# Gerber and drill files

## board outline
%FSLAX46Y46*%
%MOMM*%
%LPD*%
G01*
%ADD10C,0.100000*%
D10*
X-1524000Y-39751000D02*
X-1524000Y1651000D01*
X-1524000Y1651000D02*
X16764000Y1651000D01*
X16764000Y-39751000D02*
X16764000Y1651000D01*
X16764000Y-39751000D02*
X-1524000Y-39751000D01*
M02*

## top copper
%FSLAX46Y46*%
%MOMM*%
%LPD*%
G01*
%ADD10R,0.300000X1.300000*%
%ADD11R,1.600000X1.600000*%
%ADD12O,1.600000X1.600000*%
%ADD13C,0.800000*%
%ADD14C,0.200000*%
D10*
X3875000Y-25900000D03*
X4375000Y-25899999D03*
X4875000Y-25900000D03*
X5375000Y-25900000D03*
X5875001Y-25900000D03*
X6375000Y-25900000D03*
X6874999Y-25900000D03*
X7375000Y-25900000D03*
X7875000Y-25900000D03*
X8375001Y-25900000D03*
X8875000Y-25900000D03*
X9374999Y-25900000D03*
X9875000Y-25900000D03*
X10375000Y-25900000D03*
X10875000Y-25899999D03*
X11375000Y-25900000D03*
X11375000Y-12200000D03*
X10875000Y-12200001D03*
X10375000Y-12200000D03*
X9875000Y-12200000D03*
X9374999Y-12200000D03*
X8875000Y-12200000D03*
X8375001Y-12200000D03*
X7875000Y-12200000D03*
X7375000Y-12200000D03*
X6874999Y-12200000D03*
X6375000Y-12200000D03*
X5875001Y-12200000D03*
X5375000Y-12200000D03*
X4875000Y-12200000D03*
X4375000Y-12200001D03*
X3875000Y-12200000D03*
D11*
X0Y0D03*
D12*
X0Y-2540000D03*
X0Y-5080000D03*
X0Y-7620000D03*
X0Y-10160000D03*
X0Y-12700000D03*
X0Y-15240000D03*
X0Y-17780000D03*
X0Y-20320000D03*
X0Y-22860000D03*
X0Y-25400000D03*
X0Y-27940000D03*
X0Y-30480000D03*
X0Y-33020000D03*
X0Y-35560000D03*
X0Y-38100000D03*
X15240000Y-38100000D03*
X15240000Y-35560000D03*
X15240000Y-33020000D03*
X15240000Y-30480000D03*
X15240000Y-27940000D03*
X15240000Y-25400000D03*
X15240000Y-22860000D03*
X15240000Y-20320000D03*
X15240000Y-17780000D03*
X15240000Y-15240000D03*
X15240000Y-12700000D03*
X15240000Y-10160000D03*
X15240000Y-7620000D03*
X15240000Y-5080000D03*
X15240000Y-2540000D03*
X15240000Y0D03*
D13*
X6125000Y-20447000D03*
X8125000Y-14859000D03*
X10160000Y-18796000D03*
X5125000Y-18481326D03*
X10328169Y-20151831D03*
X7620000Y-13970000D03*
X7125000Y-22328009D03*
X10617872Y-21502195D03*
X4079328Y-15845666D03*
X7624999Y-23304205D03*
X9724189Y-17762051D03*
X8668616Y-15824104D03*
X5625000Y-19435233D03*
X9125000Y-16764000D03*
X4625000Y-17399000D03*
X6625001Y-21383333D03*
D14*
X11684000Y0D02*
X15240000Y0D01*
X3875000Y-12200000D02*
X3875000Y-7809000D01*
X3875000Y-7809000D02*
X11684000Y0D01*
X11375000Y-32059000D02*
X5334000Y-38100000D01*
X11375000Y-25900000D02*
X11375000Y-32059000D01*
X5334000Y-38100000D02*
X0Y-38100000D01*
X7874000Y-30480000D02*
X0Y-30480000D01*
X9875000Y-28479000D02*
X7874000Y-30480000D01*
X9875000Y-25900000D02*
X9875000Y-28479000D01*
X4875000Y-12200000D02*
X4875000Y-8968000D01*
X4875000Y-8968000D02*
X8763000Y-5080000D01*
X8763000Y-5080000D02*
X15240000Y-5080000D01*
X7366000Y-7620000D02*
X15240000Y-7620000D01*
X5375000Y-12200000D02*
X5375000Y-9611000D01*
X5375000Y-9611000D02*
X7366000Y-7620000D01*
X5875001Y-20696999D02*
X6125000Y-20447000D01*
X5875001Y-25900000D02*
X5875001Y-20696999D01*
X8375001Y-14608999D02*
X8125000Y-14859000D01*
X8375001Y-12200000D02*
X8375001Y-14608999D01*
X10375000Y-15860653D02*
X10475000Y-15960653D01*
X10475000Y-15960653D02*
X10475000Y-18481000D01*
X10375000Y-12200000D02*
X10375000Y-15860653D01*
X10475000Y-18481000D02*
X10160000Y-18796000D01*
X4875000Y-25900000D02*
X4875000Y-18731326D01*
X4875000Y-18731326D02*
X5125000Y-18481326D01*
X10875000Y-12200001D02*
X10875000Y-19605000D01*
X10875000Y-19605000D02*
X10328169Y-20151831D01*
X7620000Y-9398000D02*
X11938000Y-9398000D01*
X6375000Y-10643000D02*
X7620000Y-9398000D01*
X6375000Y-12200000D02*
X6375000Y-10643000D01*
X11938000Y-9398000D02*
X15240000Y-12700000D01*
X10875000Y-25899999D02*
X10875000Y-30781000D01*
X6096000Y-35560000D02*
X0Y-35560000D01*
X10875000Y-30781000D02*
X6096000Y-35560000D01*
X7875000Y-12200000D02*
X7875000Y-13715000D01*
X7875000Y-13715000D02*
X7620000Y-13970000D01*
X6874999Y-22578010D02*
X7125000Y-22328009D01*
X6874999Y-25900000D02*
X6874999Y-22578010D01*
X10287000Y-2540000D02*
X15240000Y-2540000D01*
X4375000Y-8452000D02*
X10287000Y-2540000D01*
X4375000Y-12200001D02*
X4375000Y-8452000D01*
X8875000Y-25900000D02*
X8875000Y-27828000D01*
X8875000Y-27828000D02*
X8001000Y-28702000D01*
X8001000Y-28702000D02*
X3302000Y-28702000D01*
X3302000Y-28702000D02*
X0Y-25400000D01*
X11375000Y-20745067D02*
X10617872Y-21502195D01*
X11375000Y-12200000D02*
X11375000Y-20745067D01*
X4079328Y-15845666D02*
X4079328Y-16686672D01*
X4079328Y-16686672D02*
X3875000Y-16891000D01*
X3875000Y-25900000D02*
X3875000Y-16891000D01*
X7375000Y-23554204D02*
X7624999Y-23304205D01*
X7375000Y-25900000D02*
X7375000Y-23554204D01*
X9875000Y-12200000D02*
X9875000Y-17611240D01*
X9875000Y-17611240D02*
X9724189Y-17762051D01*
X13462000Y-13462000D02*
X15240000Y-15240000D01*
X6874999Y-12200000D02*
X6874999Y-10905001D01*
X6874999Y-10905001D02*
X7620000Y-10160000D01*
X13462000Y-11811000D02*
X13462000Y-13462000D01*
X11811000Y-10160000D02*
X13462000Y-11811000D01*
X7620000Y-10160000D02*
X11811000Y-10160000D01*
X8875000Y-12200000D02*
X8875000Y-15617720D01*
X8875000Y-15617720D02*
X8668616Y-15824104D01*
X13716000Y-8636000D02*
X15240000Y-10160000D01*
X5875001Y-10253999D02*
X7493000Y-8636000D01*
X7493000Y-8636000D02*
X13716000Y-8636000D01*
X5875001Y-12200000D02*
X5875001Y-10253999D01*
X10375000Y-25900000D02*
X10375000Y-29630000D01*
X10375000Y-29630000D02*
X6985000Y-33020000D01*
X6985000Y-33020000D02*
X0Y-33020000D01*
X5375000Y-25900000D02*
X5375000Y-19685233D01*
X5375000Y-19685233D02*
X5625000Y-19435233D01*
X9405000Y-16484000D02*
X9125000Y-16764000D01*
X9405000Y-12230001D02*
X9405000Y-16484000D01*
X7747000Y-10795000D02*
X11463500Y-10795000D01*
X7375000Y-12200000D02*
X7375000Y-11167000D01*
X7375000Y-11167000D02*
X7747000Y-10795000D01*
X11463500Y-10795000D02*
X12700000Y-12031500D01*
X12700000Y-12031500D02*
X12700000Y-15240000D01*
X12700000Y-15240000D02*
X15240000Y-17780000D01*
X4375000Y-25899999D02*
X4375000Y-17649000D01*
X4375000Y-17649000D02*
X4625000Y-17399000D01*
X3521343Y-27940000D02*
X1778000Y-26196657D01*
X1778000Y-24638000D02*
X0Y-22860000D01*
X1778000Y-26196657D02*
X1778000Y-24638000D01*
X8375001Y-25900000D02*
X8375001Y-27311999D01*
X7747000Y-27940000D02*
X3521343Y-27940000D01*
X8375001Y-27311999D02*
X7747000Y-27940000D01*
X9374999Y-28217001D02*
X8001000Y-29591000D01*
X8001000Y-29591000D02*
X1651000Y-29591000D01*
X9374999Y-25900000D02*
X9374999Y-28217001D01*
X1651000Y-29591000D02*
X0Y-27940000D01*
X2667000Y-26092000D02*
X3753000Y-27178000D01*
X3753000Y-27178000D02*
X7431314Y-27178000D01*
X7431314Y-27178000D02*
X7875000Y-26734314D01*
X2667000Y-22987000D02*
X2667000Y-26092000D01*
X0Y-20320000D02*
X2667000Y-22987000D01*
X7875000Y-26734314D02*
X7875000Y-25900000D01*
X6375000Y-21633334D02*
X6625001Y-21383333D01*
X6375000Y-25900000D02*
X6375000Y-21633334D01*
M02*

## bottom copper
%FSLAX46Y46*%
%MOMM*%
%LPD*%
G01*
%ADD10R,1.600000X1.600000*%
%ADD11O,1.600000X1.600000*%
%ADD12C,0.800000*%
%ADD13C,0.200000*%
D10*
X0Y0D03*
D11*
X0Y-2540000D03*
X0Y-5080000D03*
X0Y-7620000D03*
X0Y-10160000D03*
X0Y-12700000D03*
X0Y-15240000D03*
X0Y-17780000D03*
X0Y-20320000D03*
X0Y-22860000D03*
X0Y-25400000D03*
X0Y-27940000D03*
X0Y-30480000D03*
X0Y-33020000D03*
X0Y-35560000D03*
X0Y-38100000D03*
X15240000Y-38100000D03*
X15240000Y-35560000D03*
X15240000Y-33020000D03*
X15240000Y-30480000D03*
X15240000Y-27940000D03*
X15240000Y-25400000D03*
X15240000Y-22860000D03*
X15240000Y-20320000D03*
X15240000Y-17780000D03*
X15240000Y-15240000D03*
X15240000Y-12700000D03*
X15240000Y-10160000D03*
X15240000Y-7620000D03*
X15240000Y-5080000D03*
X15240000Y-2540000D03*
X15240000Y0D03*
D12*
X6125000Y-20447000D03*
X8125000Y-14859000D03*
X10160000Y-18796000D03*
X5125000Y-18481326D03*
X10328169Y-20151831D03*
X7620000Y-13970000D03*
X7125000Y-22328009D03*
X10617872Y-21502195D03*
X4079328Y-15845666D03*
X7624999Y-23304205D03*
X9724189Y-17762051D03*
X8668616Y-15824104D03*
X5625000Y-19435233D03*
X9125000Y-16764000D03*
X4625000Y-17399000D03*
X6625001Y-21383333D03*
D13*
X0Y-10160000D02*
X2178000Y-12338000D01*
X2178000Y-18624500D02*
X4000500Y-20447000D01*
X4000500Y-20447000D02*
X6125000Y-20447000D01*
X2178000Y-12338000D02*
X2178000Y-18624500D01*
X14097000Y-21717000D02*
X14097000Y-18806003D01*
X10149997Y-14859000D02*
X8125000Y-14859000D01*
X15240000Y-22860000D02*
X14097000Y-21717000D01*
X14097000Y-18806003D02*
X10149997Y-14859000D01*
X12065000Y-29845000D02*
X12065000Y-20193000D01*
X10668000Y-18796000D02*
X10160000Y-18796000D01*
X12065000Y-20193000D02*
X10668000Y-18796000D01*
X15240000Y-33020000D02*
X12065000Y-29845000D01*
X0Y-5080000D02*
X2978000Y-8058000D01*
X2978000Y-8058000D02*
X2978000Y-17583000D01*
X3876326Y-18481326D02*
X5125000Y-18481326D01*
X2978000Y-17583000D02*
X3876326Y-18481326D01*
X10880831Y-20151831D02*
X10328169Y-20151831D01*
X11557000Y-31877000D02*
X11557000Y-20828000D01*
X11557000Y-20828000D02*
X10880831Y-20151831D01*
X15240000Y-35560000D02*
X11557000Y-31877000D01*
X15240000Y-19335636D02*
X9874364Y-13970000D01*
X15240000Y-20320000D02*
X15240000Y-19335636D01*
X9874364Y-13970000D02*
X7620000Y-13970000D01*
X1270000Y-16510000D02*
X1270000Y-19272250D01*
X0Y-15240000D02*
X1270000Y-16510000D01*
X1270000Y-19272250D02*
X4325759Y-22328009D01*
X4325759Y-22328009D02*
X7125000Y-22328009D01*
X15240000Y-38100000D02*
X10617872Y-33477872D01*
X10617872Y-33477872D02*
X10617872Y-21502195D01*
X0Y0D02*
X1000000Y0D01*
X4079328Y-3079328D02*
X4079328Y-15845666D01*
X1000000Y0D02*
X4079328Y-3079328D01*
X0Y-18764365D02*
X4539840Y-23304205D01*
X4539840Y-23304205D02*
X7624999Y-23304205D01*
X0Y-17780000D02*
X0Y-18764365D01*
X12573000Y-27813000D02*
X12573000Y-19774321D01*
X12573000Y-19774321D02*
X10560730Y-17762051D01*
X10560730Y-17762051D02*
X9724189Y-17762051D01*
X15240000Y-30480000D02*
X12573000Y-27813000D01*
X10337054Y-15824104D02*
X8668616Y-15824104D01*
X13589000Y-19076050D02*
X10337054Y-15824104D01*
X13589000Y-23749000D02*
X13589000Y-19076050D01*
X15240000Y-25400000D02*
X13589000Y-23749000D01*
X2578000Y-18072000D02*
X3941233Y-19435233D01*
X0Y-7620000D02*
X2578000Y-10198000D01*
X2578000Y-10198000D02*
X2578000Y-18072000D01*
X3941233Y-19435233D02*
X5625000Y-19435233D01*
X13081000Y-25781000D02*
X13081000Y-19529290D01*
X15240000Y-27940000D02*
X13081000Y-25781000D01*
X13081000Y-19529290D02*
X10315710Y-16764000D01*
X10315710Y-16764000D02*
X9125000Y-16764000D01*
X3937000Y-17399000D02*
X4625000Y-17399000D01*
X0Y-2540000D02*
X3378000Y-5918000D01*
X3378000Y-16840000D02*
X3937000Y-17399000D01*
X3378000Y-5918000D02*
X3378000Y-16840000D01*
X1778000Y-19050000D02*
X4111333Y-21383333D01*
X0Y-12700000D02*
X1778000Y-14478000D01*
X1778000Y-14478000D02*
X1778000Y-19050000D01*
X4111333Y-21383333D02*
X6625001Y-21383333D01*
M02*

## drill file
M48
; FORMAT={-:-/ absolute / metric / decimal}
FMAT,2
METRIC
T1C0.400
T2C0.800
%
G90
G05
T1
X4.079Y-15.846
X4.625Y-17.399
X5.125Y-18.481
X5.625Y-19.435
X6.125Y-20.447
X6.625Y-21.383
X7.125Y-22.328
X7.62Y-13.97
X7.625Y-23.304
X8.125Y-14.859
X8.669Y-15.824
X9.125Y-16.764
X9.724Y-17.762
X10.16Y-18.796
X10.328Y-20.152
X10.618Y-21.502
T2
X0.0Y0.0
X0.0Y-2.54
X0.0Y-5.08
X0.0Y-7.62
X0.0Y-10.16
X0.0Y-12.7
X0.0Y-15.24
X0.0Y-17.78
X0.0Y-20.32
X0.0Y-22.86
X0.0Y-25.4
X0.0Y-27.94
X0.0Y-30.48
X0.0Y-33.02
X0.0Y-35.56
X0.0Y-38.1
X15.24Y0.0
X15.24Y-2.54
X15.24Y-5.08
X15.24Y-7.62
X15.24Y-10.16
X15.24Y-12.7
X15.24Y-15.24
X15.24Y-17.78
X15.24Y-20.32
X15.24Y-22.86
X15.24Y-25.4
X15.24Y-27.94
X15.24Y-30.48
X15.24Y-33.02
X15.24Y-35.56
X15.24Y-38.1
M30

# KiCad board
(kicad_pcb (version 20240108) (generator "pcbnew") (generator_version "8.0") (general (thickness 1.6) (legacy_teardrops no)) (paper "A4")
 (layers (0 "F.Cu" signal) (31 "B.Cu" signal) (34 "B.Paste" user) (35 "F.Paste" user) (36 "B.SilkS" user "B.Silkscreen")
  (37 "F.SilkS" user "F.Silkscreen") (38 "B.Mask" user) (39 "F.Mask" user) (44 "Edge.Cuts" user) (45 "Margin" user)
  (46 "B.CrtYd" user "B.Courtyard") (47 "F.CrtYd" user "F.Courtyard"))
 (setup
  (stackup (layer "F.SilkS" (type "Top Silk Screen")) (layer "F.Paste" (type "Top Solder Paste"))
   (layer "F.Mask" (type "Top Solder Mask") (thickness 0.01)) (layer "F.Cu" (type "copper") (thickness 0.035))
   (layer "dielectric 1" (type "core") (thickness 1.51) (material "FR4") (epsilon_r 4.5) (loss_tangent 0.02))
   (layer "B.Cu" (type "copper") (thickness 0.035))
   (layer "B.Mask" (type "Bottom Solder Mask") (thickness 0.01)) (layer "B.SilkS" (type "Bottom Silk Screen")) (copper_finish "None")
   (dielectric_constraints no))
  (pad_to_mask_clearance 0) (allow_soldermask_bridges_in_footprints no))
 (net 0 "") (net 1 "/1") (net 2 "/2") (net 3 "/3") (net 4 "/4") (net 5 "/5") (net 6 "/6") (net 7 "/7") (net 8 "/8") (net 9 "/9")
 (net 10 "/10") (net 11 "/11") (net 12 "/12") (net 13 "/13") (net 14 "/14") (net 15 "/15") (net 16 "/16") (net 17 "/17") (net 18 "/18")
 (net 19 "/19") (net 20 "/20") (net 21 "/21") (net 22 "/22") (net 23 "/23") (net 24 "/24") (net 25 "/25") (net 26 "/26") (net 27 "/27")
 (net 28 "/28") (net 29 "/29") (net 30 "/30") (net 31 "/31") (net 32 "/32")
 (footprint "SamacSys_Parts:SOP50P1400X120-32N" (layer "F.Cu") (at 7.625 19.05 90)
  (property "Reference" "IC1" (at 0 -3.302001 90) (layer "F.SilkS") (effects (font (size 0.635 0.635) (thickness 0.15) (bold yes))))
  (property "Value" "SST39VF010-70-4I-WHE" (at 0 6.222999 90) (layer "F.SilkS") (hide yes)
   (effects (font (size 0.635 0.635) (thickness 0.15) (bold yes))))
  (pad "1" smd rect (at -6.85 -3.75 180) (size 0.3 1.3) (layers "F.Cu" "F.Paste" "F.Mask") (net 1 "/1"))
  (pad "2" smd rect (at -6.849999 -3.25 180) (size 0.3 1.3) (layers "F.Cu" "F.Paste" "F.Mask") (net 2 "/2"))
  (pad "3" smd rect (at -6.85 -2.75 180) (size 0.3 1.3) (layers "F.Cu" "F.Paste" "F.Mask") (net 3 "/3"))
  (pad "4" smd rect (at -6.85 -2.25 180) (size 0.3 1.3) (layers "F.Cu" "F.Paste" "F.Mask") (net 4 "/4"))
  (pad "5" smd rect (at -6.85 -1.749999 180) (size 0.3 1.3) (layers "F.Cu" "F.Paste" "F.Mask") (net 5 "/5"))
  (pad "6" smd rect (at -6.85 -1.25 180) (size 0.3 1.3) (layers "F.Cu" "F.Paste" "F.Mask") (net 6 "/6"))
  (pad "7" smd rect (at -6.85 -0.750001 180) (size 0.3 1.3) (layers "F.Cu" "F.Paste" "F.Mask") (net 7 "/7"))
  (pad "8" smd rect (at -6.85 -0.25 180) (size 0.3 1.3) (layers "F.Cu" "F.Paste" "F.Mask") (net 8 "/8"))
  (pad "9" smd rect (at -6.85 0.25 180) (size 0.3 1.3) (layers "F.Cu" "F.Paste" "F.Mask") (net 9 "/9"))
  (pad "10" smd rect (at -6.85 0.750001 180) (size 0.3 1.3) (layers "F.Cu" "F.Paste" "F.Mask") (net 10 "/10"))
  (pad "11" smd rect (at -6.85 1.25 180) (size 0.3 1.3) (layers "F.Cu" "F.Paste" "F.Mask") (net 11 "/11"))
  (pad "12" smd rect (at -6.85 1.749999 180) (size 0.3 1.3) (layers "F.Cu" "F.Paste" "F.Mask") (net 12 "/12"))
  (pad "13" smd rect (at -6.85 2.25 180) (size 0.3 1.3) (layers "F.Cu" "F.Paste" "F.Mask") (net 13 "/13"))
  (pad "14" smd rect (at -6.85 2.75 180) (size 0.3 1.3) (layers "F.Cu" "F.Paste" "F.Mask") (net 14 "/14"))
  (pad "15" smd rect (at -6.849999 3.25 180) (size 0.3 1.3) (layers "F.Cu" "F.Paste" "F.Mask") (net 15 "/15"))
  (pad "16" smd rect (at -6.85 3.75 180) (size 0.3 1.3) (layers "F.Cu" "F.Paste" "F.Mask") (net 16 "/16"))
  (pad "17" smd rect (at 6.85 3.75 180) (size 0.3 1.3) (layers "F.Cu" "F.Paste" "F.Mask") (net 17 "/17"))
  (pad "18" smd rect (at 6.849999 3.25 180) (size 0.3 1.3) (layers "F.Cu" "F.Paste" "F.Mask") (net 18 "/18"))
  (pad "19" smd rect (at 6.85 2.75 180) (size 0.3 1.3) (layers "F.Cu" "F.Paste" "F.Mask") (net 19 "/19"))
  (pad "20" smd rect (at 6.85 2.25 180) (size 0.3 1.3) (layers "F.Cu" "F.Paste" "F.Mask") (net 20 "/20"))
  (pad "21" smd rect (at 6.85 1.749999 180) (size 0.3 1.3) (layers "F.Cu" "F.Paste" "F.Mask") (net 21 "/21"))
  (pad "22" smd rect (at 6.85 1.25 180) (size 0.3 1.3) (layers "F.Cu" "F.Paste" "F.Mask") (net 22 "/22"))
  (pad "23" smd rect (at 6.85 0.750001 180) (size 0.3 1.3) (layers "F.Cu" "F.Paste" "F.Mask") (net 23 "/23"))
  (pad "24" smd rect (at 6.85 0.25 180) (size 0.3 1.3) (layers "F.Cu" "F.Paste" "F.Mask") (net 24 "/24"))
  (pad "25" smd rect (at 6.85 -0.25 180) (size 0.3 1.3) (layers "F.Cu" "F.Paste" "F.Mask") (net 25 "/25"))
  (pad "26" smd rect (at 6.85 -0.750001 180) (size 0.3 1.3) (layers "F.Cu" "F.Paste" "F.Mask") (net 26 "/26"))
  (pad "27" smd rect (at 6.85 -1.25 180) (size 0.3 1.3) (layers "F.Cu" "F.Paste" "F.Mask") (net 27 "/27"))
  (pad "28" smd rect (at 6.85 -1.749999 180) (size 0.3 1.3) (layers "F.Cu" "F.Paste" "F.Mask") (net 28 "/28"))
  (pad "29" smd rect (at 6.85 -2.25 180) (size 0.3 1.3) (layers "F.Cu" "F.Paste" "F.Mask") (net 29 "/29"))
  (pad "30" smd rect (at 6.85 -2.75 180) (size 0.3 1.3) (layers "F.Cu" "F.Paste" "F.Mask") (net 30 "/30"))
  (pad "31" smd rect (at 6.849999 -3.25 180) (size 0.3 1.3) (layers "F.Cu" "F.Paste" "F.Mask") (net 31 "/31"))
  (pad "32" smd rect (at 6.85 -3.75 180) (size 0.3 1.3) (layers "F.Cu" "F.Paste" "F.Mask") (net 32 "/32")))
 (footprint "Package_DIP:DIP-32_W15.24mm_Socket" (layer "F.Cu") (at 0 0)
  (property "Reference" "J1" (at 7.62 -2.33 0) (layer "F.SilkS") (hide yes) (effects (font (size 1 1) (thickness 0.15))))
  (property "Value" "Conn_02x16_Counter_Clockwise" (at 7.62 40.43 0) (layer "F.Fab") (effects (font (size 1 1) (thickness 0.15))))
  (pad "1" thru_hole rect (at 0 0) (size 1.6 1.6) (drill 0.8) (layers "*.Cu" "*.Mask") (remove_unused_layers no) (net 1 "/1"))
  (pad "2" thru_hole oval (at 0 2.54) (size 1.6 1.6) (drill 0.8) (layers "*.Cu" "*.Mask") (remove_unused_layers no) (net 2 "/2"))
  (pad "3" thru_hole oval (at 0 5.08) (size 1.6 1.6) (drill 0.8) (layers "*.Cu" "*.Mask") (remove_unused_layers no) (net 3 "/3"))
  (pad "4" thru_hole oval (at 0 7.62) (size 1.6 1.6) (drill 0.8) (layers "*.Cu" "*.Mask") (remove_unused_layers no) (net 4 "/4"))
  (pad "5" thru_hole oval (at 0 10.16) (size 1.6 1.6) (drill 0.8) (layers "*.Cu" "*.Mask") (remove_unused_layers no) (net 5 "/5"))
  (pad "6" thru_hole oval (at 0 12.7) (size 1.6 1.6) (drill 0.8) (layers "*.Cu" "*.Mask") (remove_unused_layers no) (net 6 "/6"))
  (pad "7" thru_hole oval (at 0 15.24) (size 1.6 1.6) (drill 0.8) (layers "*.Cu" "*.Mask") (remove_unused_layers no) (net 7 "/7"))
  (pad "8" thru_hole oval (at 0 17.78) (size 1.6 1.6) (drill 0.8) (layers "*.Cu" "*.Mask") (remove_unused_layers no) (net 8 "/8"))
  (pad "9" thru_hole oval (at 0 20.32) (size 1.6 1.6) (drill 0.8) (layers "*.Cu" "*.Mask") (remove_unused_layers no) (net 9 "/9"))
  (pad "10" thru_hole oval (at 0 22.86) (size 1.6 1.6) (drill 0.8) (layers "*.Cu" "*.Mask") (remove_unused_layers no) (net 10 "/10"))
  (pad "11" thru_hole oval (at 0 25.4) (size 1.6 1.6) (drill 0.8) (layers "*.Cu" "*.Mask") (remove_unused_layers no) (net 11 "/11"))
  (pad "12" thru_hole oval (at 0 27.94) (size 1.6 1.6) (drill 0.8) (layers "*.Cu" "*.Mask") (remove_unused_layers no) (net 12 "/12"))
  (pad "13" thru_hole oval (at 0 30.48) (size 1.6 1.6) (drill 0.8) (layers "*.Cu" "*.Mask") (remove_unused_layers no) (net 13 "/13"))
  (pad "14" thru_hole oval (at 0 33.02) (size 1.6 1.6) (drill 0.8) (layers "*.Cu" "*.Mask") (remove_unused_layers no) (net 14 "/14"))
  (pad "15" thru_hole oval (at 0 35.56) (size 1.6 1.6) (drill 0.8) (layers "*.Cu" "*.Mask") (remove_unused_layers no) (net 15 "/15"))
  (pad "16" thru_hole oval (at 0 38.1) (size 1.6 1.6) (drill 0.8) (layers "*.Cu" "*.Mask") (remove_unused_layers no) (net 16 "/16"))
  (pad "17" thru_hole oval (at 15.24 38.1) (size 1.6 1.6) (drill 0.8) (layers "*.Cu" "*.Mask") (remove_unused_layers no) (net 17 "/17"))
  (pad "18" thru_hole oval (at 15.24 35.56) (size 1.6 1.6) (drill 0.8) (layers "*.Cu" "*.Mask") (remove_unused_layers no) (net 18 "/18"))
  (pad "19" thru_hole oval (at 15.24 33.02) (size 1.6 1.6) (drill 0.8) (layers "*.Cu" "*.Mask") (remove_unused_layers no) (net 19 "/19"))
  (pad "20" thru_hole oval (at 15.24 30.48) (size 1.6 1.6) (drill 0.8) (layers "*.Cu" "*.Mask") (remove_unused_layers no) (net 20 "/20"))
  (pad "21" thru_hole oval (at 15.24 27.94) (size 1.6 1.6) (drill 0.8) (layers "*.Cu" "*.Mask") (remove_unused_layers no) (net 21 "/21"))
  (pad "22" thru_hole oval (at 15.24 25.4) (size 1.6 1.6) (drill 0.8) (layers "*.Cu" "*.Mask") (remove_unused_layers no) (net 22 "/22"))
  (pad "23" thru_hole oval (at 15.24 22.86) (size 1.6 1.6) (drill 0.8) (layers "*.Cu" "*.Mask") (remove_unused_layers no) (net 23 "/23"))
  (pad "24" thru_hole oval (at 15.24 20.32) (size 1.6 1.6) (drill 0.8) (layers "*.Cu" "*.Mask") (remove_unused_layers no) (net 24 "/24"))
  (pad "25" thru_hole oval (at 15.24 17.78) (size 1.6 1.6) (drill 0.8) (layers "*.Cu" "*.Mask") (remove_unused_layers no) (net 25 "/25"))
  (pad "26" thru_hole oval (at 15.24 15.24) (size 1.6 1.6) (drill 0.8) (layers "*.Cu" "*.Mask") (remove_unused_layers no) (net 26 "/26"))
  (pad "27" thru_hole oval (at 15.24 12.7) (size 1.6 1.6) (drill 0.8) (layers "*.Cu" "*.Mask") (remove_unused_layers no) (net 27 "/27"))
  (pad "28" thru_hole oval (at 15.24 10.16) (size 1.6 1.6) (drill 0.8) (layers "*.Cu" "*.Mask") (remove_unused_layers no) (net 28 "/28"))
  (pad "29" thru_hole oval (at 15.24 7.62) (size 1.6 1.6) (drill 0.8) (layers "*.Cu" "*.Mask") (remove_unused_layers no) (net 29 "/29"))
  (pad "30" thru_hole oval (at 15.24 5.08) (size 1.6 1.6) (drill 0.8) (layers "*.Cu" "*.Mask") (remove_unused_layers no) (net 30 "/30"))
  (pad "31" thru_hole oval (at 15.24 2.54) (size 1.6 1.6) (drill 0.8) (layers "*.Cu" "*.Mask") (remove_unused_layers no) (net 31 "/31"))
  (pad "32" thru_hole oval (at 15.24 0) (size 1.6 1.6) (drill 0.8) (layers "*.Cu" "*.Mask") (remove_unused_layers no) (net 32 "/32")))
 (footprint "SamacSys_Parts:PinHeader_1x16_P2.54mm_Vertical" (layer "B.Cu") (at 0 0 180)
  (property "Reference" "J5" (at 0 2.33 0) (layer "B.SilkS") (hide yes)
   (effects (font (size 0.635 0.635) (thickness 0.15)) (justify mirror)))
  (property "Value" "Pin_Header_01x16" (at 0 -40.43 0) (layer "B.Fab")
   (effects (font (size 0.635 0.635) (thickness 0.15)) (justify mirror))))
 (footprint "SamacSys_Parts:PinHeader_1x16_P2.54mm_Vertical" (layer "B.Cu") (at 15.24 0 180)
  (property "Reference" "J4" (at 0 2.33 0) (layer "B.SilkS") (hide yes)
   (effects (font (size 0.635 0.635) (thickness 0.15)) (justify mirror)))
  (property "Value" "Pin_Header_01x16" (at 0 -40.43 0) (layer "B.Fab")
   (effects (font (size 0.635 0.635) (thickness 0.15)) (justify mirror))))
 (gr_line (start -1.524 39.751) (end -1.524 -1.651) (stroke (width 0.1) (type solid)) (layer "Edge.Cuts"))
 (gr_line (start -1.524 -1.651) (end 16.764 -1.651) (stroke (width 0.1) (type solid)) (layer "Edge.Cuts"))
 (gr_line (start 16.764 39.751) (end 16.764 -1.651) (stroke (width 0.1) (type solid)) (layer "Edge.Cuts"))
 (gr_line (start 16.764 39.751) (end -1.524 39.751) (stroke (width 0.1) (type solid)) (layer "Edge.Cuts"))
 (segment (start 11.684 0) (end 15.24 0) (width 0.2) (layer "F.Cu") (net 32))
 (segment (start 3.875 12.2) (end 3.875 7.809) (width 0.2) (layer "F.Cu") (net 32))
 (segment (start 3.875 7.809) (end 11.684 0) (width 0.2) (layer "F.Cu") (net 32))
 (segment (start 11.375 32.059) (end 5.334 38.1) (width 0.2) (layer "F.Cu") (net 16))
 (segment (start 11.375 25.9) (end 11.375 32.059) (width 0.2) (layer "F.Cu") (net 16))
 (segment (start 5.334 38.1) (end 0 38.1) (width 0.2) (layer "F.Cu") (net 16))
 (segment (start 7.874 30.48) (end 0 30.48) (width 0.2) (layer "F.Cu") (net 13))
 (segment (start 9.875 28.479) (end 7.874 30.48) (width 0.2) (layer "F.Cu") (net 13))
 (segment (start 9.875 25.9) (end 9.875 28.479) (width 0.2) (layer "F.Cu") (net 13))
 (segment (start 4.875 12.2) (end 4.875 8.968) (width 0.2) (layer "F.Cu") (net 30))
 (segment (start 4.875 8.968) (end 8.763 5.08) (width 0.2) (layer "F.Cu") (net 30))
 (segment (start 8.763 5.08) (end 15.24 5.08) (width 0.2) (layer "F.Cu") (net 30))
 (segment (start 7.366 7.62) (end 15.24 7.62) (width 0.2) (layer "F.Cu") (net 29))
 (segment (start 5.375 12.2) (end 5.375 9.611) (width 0.2) (layer "F.Cu") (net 29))
 (segment (start 5.375 9.611) (end 7.366 7.62) (width 0.2) (layer "F.Cu") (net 29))
 (segment (start 5.875001 20.696999) (end 6.125 20.447) (width 0.2) (layer "F.Cu") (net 5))
 (segment (start 5.875001 25.9) (end 5.875001 20.696999) (width 0.2) (layer "F.Cu") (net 5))
 (via (at 6.125 20.447) (size 0.8) (drill 0.4) (layers "F.Cu" "B.Cu") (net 5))
 (segment (start 0 10.16) (end 2.178 12.338) (width 0.2) (layer "B.Cu") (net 5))
 (segment (start 2.178 18.6245) (end 4.0005 20.447) (width 0.2) (layer "B.Cu") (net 5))
 (segment (start 4.0005 20.447) (end 6.125 20.447) (width 0.2) (layer "B.Cu") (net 5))
 (segment (start 2.178 12.338) (end 2.178 18.6245) (width 0.2) (layer "B.Cu") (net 5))
 (segment (start 8.375001 14.608999) (end 8.125 14.859) (width 0.2) (layer "F.Cu") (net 23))
 (segment (start 8.375001 12.2) (end 8.375001 14.608999) (width 0.2) (layer "F.Cu") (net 23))
 (via (at 8.125 14.859) (size 0.8) (drill 0.4) (layers "F.Cu" "B.Cu") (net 23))
 (segment (start 14.097 21.717) (end 14.097 18.806003) (width 0.2) (layer "B.Cu") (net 23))
 (segment (start 10.149997 14.859) (end 8.125 14.859) (width 0.2) (layer "B.Cu") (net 23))
 (segment (start 15.24 22.86) (end 14.097 21.717) (width 0.2) (layer "B.Cu") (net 23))
 (segment (start 14.097 18.806003) (end 10.149997 14.859) (width 0.2) (layer "B.Cu") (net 23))
 (segment (start 10.375 15.860653) (end 10.475 15.960653) (width 0.2) (layer "F.Cu") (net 19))
 (segment (start 10.475 15.960653) (end 10.475 18.481) (width 0.2) (layer "F.Cu") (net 19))
 (segment (start 10.375 12.2) (end 10.375 15.860653) (width 0.2) (layer "F.Cu") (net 19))
 (segment (start 10.475 18.481) (end 10.16 18.796) (width 0.2) (layer "F.Cu") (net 19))
 (via (at 10.16 18.796) (size 0.8) (drill 0.4) (layers "F.Cu" "B.Cu") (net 19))
 (segment (start 12.065 29.845) (end 12.065 20.193) (width 0.2) (layer "B.Cu") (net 19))
 (segment (start 10.668 18.796) (end 10.16 18.796) (width 0.2) (layer "B.Cu") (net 19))
 (segment (start 12.065 20.193) (end 10.668 18.796) (width 0.2) (layer "B.Cu") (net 19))
 (segment (start 15.24 33.02) (end 12.065 29.845) (width 0.2) (layer "B.Cu") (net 19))
 (segment (start 4.875 25.9) (end 4.875 18.731326) (width 0.2) (layer "F.Cu") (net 3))
 (segment (start 4.875 18.731326) (end 5.125 18.481326) (width 0.2) (layer "F.Cu") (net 3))
 (via (at 5.125 18.481326) (size 0.8) (drill 0.4) (layers "F.Cu" "B.Cu") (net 3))
 (segment (start 0 5.08) (end 2.978 8.058) (width 0.2) (layer "B.Cu") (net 3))
 (segment (start 2.978 8.058) (end 2.978 17.583) (width 0.2) (layer "B.Cu") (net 3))
 (segment (start 3.876326 18.481326) (end 5.125 18.481326) (width 0.2) (layer "B.Cu") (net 3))
 (segment (start 2.978 17.583) (end 3.876326 18.481326) (width 0.2) (layer "B.Cu") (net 3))
 (segment (start 10.875 12.200001) (end 10.875 19.605) (width 0.2) (layer "F.Cu") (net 18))
 (segment (start 10.875 19.605) (end 10.328169 20.151831) (width 0.2) (layer "F.Cu") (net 18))
 (via (at 10.328169 20.151831) (size 0.8) (drill 0.4) (layers "F.Cu" "B.Cu") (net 18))
 (segment (start 10.880831 20.151831) (end 10.328169 20.151831) (width 0.2) (layer "B.Cu") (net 18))
 (segment (start 11.557 31.877) (end 11.557 20.828) (width 0.2) (layer "B.Cu") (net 18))
 (segment (start 11.557 20.828) (end 10.880831 20.151831) (width 0.2) (layer "B.Cu") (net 18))
 (segment (start 15.24 35.56) (end 11.557 31.877) (width 0.2) (layer "B.Cu") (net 18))
 (segment (start 7.62 9.398) (end 11.938 9.398) (width 0.2) (layer "F.Cu") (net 27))
 (segment (start 6.375 10.643) (end 7.62 9.398) (width 0.2) (layer "F.Cu") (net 27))
 (segment (start 6.375 12.2) (end 6.375 10.643) (width 0.2) (layer "F.Cu") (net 27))
 (segment (start 11.938 9.398) (end 15.24 12.7) (width 0.2) (layer "F.Cu") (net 27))
 (segment (start 10.875 25.899999) (end 10.875 30.781) (width 0.2) (layer "F.Cu") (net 15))
 (segment (start 6.096 35.56) (end 0 35.56) (width 0.2) (layer "F.Cu") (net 15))
 (segment (start 10.875 30.781) (end 6.096 35.56) (width 0.2) (layer "F.Cu") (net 15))
 (segment (start 7.875 12.2) (end 7.875 13.715) (width 0.2) (layer "F.Cu") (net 24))
 (segment (start 7.875 13.715) (end 7.62 13.97) (width 0.2) (layer "F.Cu") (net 24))
 (via (at 7.62 13.97) (size 0.8) (drill 0.4) (layers "F.Cu" "B.Cu") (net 24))
 (segment (start 15.24 19.335636) (end 9.874364 13.97) (width 0.2) (layer "B.Cu") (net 24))
 (segment (start 15.24 20.32) (end 15.24 19.335636) (width 0.2) (layer "B.Cu") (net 24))
 (segment (start 9.874364 13.97) (end 7.62 13.97) (width 0.2) (layer "B.Cu") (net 24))
 (segment (start 6.874999 22.57801) (end 7.125 22.328009) (width 0.2) (layer "F.Cu") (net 7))
 (segment (start 6.874999 25.9) (end 6.874999 22.57801) (width 0.2) (layer "F.Cu") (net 7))
 (via (at 7.125 22.328009) (size 0.8) (drill 0.4) (layers "F.Cu" "B.Cu") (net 7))
 (segment (start 1.27 16.51) (end 1.27 19.27225) (width 0.2) (layer "B.Cu") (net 7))
 (segment (start 0 15.24) (end 1.27 16.51) (width 0.2) (layer "B.Cu") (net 7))
 (segment (start 1.27 19.27225) (end 4.325759 22.328009) (width 0.2) (layer "B.Cu") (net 7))
 (segment (start 4.325759 22.328009) (end 7.125 22.328009) (width 0.2) (layer "B.Cu") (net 7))
 (segment (start 10.287 2.54) (end 15.24 2.54) (width 0.2) (layer "F.Cu") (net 31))
 (segment (start 4.375 8.452) (end 10.287 2.54) (width 0.2) (layer "F.Cu") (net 31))
 (segment (start 4.375 12.200001) (end 4.375 8.452) (width 0.2) (layer "F.Cu") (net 31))
 (segment (start 8.875 25.9) (end 8.875 27.828) (width 0.2) (layer "F.Cu") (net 11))
 (segment (start 8.875 27.828) (end 8.001 28.702) (width 0.2) (layer "F.Cu") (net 11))
 (segment (start 8.001 28.702) (end 3.302 28.702) (width 0.2) (layer "F.Cu") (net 11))
 (segment (start 3.302 28.702) (end 0 25.4) (width 0.2) (layer "F.Cu") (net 11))
 (segment (start 11.375 20.745067) (end 10.617872 21.502195) (width 0.2) (layer "F.Cu") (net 17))
 (segment (start 11.375 12.2) (end 11.375 20.745067) (width 0.2) (layer "F.Cu") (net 17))
 (via (at 10.617872 21.502195) (size 0.8) (drill 0.4) (layers "F.Cu" "B.Cu") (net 17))
 (segment (start 15.24 38.1) (end 10.617872 33.477872) (width 0.2) (layer "B.Cu") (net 17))
 (segment (start 10.617872 33.477872) (end 10.617872 21.502195) (width 0.2) (layer "B.Cu") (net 17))
 (segment (start 4.079328 15.845666) (end 4.079328 16.686672) (width 0.2) (layer "F.Cu") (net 1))
 (segment (start 4.079328 16.686672) (end 3.875 16.891) (width 0.2) (layer "F.Cu") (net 1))
 (segment (start 3.875 25.9) (end 3.875 16.891) (width 0.2) (layer "F.Cu") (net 1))
 (via (at 4.079328 15.845666) (size 0.8) (drill 0.4) (layers "F.Cu" "B.Cu") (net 1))
 (segment (start 0 0) (end 1 0) (width 0.2) (layer "B.Cu") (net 1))
 (segment (start 4.079328 3.079328) (end 4.079328 15.845666) (width 0.2) (layer "B.Cu") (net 1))
 (segment (start 1 0) (end 4.079328 3.079328) (width 0.2) (layer "B.Cu") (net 1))
 (segment (start 7.375 23.554204) (end 7.624999 23.304205) (width 0.2) (layer "F.Cu") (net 8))
 (segment (start 7.375 25.9) (end 7.375 23.554204) (width 0.2) (layer "F.Cu") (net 8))
 (via (at 7.624999 23.304205) (size 0.8) (drill 0.4) (layers "F.Cu" "B.Cu") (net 8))
 (segment (start 0 18.764365) (end 4.53984 23.304205) (width 0.2) (layer "B.Cu") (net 8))
 (segment (start 4.53984 23.304205) (end 7.624999 23.304205) (width 0.2) (layer "B.Cu") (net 8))
 (segment (start 0 17.78) (end 0 18.764365) (width 0.2) (layer "B.Cu") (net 8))
 (segment (start 9.875 12.2) (end 9.875 17.61124) (width 0.2) (layer "F.Cu") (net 20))
 (segment (start 9.875 17.61124) (end 9.724189 17.762051) (width 0.2) (layer "F.Cu") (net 20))
 (via (at 9.724189 17.762051) (size 0.8) (drill 0.4) (layers "F.Cu" "B.Cu") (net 20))
 (segment (start 12.573 27.813) (end 12.573 19.774321) (width 0.2) (layer "B.Cu") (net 20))
 (segment (start 12.573 19.774321) (end 10.56073 17.762051) (width 0.2) (layer "B.Cu") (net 20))
 (segment (start 10.56073 17.762051) (end 9.724189 17.762051) (width 0.2) (layer "B.Cu") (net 20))
 (segment (start 15.24 30.48) (end 12.573 27.813) (width 0.2) (layer "B.Cu") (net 20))
 (segment (start 13.462 13.462) (end 15.24 15.24) (width 0.2) (layer "F.Cu") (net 26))
 (segment (start 6.874999 12.2) (end 6.874999 10.905001) (width 0.2) (layer "F.Cu") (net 26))
 (segment (start 6.874999 10.905001) (end 7.62 10.16) (width 0.2) (layer "F.Cu") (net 26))
 (segment (start 13.462 11.811) (end 13.462 13.462) (width 0.2) (layer "F.Cu") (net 26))
 (segment (start 11.811 10.16) (end 13.462 11.811) (width 0.2) (layer "F.Cu") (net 26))
 (segment (start 7.62 10.16) (end 11.811 10.16) (width 0.2) (layer "F.Cu") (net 26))
 (segment (start 8.875 12.2) (end 8.875 15.61772) (width 0.2) (layer "F.Cu") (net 22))
 (segment (start 8.875 15.61772) (end 8.668616 15.824104) (width 0.2) (layer "F.Cu") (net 22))
 (via (at 8.668616 15.824104) (size 0.8) (drill 0.4) (layers "F.Cu" "B.Cu") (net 22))
 (segment (start 10.337054 15.824104) (end 8.668616 15.824104) (width 0.2) (layer "B.Cu") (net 22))
 (segment (start 13.589 19.07605) (end 10.337054 15.824104) (width 0.2) (layer "B.Cu") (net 22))
 (segment (start 13.589 23.749) (end 13.589 19.07605) (width 0.2) (layer "B.Cu") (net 22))
 (segment (start 15.24 25.4) (end 13.589 23.749) (width 0.2) (layer "B.Cu") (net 22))
 (segment (start 13.716 8.636) (end 15.24 10.16) (width 0.2) (layer "F.Cu") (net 28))
 (segment (start 5.875001 10.253999) (end 7.493 8.636) (width 0.2) (layer "F.Cu") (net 28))
 (segment (start 7.493 8.636) (end 13.716 8.636) (width 0.2) (layer "F.Cu") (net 28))
 (segment (start 5.875001 12.2) (end 5.875001 10.253999) (width 0.2) (layer "F.Cu") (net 28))
 (segment (start 10.375 25.9) (end 10.375 29.63) (width 0.2) (layer "F.Cu") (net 14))
 (segment (start 10.375 29.63) (end 6.985 33.02) (width 0.2) (layer "F.Cu") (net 14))
 (segment (start 6.985 33.02) (end 0 33.02) (width 0.2) (layer "F.Cu") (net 14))
 (segment (start 5.375 25.9) (end 5.375 19.685233) (width 0.2) (layer "F.Cu") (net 4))
 (segment (start 5.375 19.685233) (end 5.625 19.435233) (width 0.2) (layer "F.Cu") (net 4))
 (via (at 5.625 19.435233) (size 0.8) (drill 0.4) (layers "F.Cu" "B.Cu") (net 4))
 (segment (start 2.578 18.072) (end 3.941233 19.435233) (width 0.2) (layer "B.Cu") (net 4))
 (segment (start 0 7.62) (end 2.578 10.198) (width 0.2) (layer "B.Cu") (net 4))
 (segment (start 2.578 10.198) (end 2.578 18.072) (width 0.2) (layer "B.Cu") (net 4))
 (segment (start 3.941233 19.435233) (end 5.625 19.435233) (width 0.2) (layer "B.Cu") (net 4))
 (segment (start 9.405 16.484) (end 9.125 16.764) (width 0.2) (layer "F.Cu") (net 21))
 (segment (start 9.405 12.230001) (end 9.405 16.484) (width 0.2) (layer "F.Cu") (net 21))
 (via (at 9.125 16.764) (size 0.8) (drill 0.4) (layers "F.Cu" "B.Cu") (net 21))
 (segment (start 13.081 25.781) (end 13.081 19.52929) (width 0.2) (layer "B.Cu") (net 21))
 (segment (start 15.24 27.94) (end 13.081 25.781) (width 0.2) (layer "B.Cu") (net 21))
 (segment (start 13.081 19.52929) (end 10.31571 16.764) (width 0.2) (layer "B.Cu") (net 21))
 (segment (start 10.31571 16.764) (end 9.125 16.764) (width 0.2) (layer "B.Cu") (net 21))
 (segment (start 7.747 10.795) (end 11.4635 10.795) (width 0.2) (layer "F.Cu") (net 25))
 (segment (start 7.375 12.2) (end 7.375 11.167) (width 0.2) (layer "F.Cu") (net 25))
 (segment (start 7.375 11.167) (end 7.747 10.795) (width 0.2) (layer "F.Cu") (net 25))
 (segment (start 11.4635 10.795) (end 12.7 12.0315) (width 0.2) (layer "F.Cu") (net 25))
 (segment (start 12.7 12.0315) (end 12.7 15.24) (width 0.2) (layer "F.Cu") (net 25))
 (segment (start 12.7 15.24) (end 15.24 17.78) (width 0.2) (layer "F.Cu") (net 25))
 (segment (start 4.375 25.899999) (end 4.375 17.649) (width 0.2) (layer "F.Cu") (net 2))
 (segment (start 4.375 17.649) (end 4.625 17.399) (width 0.2) (layer "F.Cu") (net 2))
 (via (at 4.625 17.399) (size 0.8) (drill 0.4) (layers "F.Cu" "B.Cu") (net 2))
 (segment (start 3.937 17.399) (end 4.625 17.399) (width 0.2) (layer "B.Cu") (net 2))
 (segment (start 0 2.54) (end 3.378 5.918) (width 0.2) (layer "B.Cu") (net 2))
 (segment (start 3.378 16.84) (end 3.937 17.399) (width 0.2) (layer "B.Cu") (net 2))
 (segment (start 3.378 5.918) (end 3.378 16.84) (width 0.2) (layer "B.Cu") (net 2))
 (segment (start 3.521343 27.94) (end 1.778 26.196657) (width 0.2) (layer "F.Cu") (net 10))
 (segment (start 1.778 24.638) (end 0 22.86) (width 0.2) (layer "F.Cu") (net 10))
 (segment (start 1.778 26.196657) (end 1.778 24.638) (width 0.2) (layer "F.Cu") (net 10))
 (segment (start 8.375001 25.9) (end 8.375001 27.311999) (width 0.2) (layer "F.Cu") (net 10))
 (segment (start 7.747 27.94) (end 3.521343 27.94) (width 0.2) (layer "F.Cu") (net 10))
 (segment (start 8.375001 27.311999) (end 7.747 27.94) (width 0.2) (layer "F.Cu") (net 10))
 (segment (start 9.374999 28.217001) (end 8.001 29.591) (width 0.2) (layer "F.Cu") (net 12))
 (segment (start 8.001 29.591) (end 1.651 29.591) (width 0.2) (layer "F.Cu") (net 12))
 (segment (start 9.374999 25.9) (end 9.374999 28.217001) (width 0.2) (layer "F.Cu") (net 12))
 (segment (start 1.651 29.591) (end 0 27.94) (width 0.2) (layer "F.Cu") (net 12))
 (segment (start 2.667 26.092) (end 3.753 27.178) (width 0.2) (layer "F.Cu") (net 9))
 (segment (start 3.753 27.178) (end 7.431314 27.178) (width 0.2) (layer "F.Cu") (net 9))
 (segment (start 7.431314 27.178) (end 7.875 26.734314) (width 0.2) (layer "F.Cu") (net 9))
 (segment (start 2.667 22.987) (end 2.667 26.092) (width 0.2) (layer "F.Cu") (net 9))
 (segment (start 0 20.32) (end 2.667 22.987) (width 0.2) (layer "F.Cu") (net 9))
 (segment (start 7.875 26.734314) (end 7.875 25.9) (width 0.2) (layer "F.Cu") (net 9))
 (segment (start 6.375 21.633334) (end 6.625001 21.383333) (width 0.2) (layer "F.Cu") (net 6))
 (segment (start 6.375 25.9) (end 6.375 21.633334) (width 0.2) (layer "F.Cu") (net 6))
 (via (at 6.625001 21.383333) (size 0.8) (drill 0.4) (layers "F.Cu" "B.Cu") (free yes) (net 6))
 (segment (start 1.778 19.05) (end 4.111333 21.383333) (width 0.2) (layer "B.Cu") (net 6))
 (segment (start 0 12.7) (end 1.778 14.478) (width 0.2) (layer "B.Cu") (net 6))
 (segment (start 1.778 14.478) (end 1.778 19.05) (width 0.2) (layer "B.Cu") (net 6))
 (segment (start 4.111333 21.383333) (end 6.625001 21.383333) (width 0.2) (layer "B.Cu") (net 6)))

